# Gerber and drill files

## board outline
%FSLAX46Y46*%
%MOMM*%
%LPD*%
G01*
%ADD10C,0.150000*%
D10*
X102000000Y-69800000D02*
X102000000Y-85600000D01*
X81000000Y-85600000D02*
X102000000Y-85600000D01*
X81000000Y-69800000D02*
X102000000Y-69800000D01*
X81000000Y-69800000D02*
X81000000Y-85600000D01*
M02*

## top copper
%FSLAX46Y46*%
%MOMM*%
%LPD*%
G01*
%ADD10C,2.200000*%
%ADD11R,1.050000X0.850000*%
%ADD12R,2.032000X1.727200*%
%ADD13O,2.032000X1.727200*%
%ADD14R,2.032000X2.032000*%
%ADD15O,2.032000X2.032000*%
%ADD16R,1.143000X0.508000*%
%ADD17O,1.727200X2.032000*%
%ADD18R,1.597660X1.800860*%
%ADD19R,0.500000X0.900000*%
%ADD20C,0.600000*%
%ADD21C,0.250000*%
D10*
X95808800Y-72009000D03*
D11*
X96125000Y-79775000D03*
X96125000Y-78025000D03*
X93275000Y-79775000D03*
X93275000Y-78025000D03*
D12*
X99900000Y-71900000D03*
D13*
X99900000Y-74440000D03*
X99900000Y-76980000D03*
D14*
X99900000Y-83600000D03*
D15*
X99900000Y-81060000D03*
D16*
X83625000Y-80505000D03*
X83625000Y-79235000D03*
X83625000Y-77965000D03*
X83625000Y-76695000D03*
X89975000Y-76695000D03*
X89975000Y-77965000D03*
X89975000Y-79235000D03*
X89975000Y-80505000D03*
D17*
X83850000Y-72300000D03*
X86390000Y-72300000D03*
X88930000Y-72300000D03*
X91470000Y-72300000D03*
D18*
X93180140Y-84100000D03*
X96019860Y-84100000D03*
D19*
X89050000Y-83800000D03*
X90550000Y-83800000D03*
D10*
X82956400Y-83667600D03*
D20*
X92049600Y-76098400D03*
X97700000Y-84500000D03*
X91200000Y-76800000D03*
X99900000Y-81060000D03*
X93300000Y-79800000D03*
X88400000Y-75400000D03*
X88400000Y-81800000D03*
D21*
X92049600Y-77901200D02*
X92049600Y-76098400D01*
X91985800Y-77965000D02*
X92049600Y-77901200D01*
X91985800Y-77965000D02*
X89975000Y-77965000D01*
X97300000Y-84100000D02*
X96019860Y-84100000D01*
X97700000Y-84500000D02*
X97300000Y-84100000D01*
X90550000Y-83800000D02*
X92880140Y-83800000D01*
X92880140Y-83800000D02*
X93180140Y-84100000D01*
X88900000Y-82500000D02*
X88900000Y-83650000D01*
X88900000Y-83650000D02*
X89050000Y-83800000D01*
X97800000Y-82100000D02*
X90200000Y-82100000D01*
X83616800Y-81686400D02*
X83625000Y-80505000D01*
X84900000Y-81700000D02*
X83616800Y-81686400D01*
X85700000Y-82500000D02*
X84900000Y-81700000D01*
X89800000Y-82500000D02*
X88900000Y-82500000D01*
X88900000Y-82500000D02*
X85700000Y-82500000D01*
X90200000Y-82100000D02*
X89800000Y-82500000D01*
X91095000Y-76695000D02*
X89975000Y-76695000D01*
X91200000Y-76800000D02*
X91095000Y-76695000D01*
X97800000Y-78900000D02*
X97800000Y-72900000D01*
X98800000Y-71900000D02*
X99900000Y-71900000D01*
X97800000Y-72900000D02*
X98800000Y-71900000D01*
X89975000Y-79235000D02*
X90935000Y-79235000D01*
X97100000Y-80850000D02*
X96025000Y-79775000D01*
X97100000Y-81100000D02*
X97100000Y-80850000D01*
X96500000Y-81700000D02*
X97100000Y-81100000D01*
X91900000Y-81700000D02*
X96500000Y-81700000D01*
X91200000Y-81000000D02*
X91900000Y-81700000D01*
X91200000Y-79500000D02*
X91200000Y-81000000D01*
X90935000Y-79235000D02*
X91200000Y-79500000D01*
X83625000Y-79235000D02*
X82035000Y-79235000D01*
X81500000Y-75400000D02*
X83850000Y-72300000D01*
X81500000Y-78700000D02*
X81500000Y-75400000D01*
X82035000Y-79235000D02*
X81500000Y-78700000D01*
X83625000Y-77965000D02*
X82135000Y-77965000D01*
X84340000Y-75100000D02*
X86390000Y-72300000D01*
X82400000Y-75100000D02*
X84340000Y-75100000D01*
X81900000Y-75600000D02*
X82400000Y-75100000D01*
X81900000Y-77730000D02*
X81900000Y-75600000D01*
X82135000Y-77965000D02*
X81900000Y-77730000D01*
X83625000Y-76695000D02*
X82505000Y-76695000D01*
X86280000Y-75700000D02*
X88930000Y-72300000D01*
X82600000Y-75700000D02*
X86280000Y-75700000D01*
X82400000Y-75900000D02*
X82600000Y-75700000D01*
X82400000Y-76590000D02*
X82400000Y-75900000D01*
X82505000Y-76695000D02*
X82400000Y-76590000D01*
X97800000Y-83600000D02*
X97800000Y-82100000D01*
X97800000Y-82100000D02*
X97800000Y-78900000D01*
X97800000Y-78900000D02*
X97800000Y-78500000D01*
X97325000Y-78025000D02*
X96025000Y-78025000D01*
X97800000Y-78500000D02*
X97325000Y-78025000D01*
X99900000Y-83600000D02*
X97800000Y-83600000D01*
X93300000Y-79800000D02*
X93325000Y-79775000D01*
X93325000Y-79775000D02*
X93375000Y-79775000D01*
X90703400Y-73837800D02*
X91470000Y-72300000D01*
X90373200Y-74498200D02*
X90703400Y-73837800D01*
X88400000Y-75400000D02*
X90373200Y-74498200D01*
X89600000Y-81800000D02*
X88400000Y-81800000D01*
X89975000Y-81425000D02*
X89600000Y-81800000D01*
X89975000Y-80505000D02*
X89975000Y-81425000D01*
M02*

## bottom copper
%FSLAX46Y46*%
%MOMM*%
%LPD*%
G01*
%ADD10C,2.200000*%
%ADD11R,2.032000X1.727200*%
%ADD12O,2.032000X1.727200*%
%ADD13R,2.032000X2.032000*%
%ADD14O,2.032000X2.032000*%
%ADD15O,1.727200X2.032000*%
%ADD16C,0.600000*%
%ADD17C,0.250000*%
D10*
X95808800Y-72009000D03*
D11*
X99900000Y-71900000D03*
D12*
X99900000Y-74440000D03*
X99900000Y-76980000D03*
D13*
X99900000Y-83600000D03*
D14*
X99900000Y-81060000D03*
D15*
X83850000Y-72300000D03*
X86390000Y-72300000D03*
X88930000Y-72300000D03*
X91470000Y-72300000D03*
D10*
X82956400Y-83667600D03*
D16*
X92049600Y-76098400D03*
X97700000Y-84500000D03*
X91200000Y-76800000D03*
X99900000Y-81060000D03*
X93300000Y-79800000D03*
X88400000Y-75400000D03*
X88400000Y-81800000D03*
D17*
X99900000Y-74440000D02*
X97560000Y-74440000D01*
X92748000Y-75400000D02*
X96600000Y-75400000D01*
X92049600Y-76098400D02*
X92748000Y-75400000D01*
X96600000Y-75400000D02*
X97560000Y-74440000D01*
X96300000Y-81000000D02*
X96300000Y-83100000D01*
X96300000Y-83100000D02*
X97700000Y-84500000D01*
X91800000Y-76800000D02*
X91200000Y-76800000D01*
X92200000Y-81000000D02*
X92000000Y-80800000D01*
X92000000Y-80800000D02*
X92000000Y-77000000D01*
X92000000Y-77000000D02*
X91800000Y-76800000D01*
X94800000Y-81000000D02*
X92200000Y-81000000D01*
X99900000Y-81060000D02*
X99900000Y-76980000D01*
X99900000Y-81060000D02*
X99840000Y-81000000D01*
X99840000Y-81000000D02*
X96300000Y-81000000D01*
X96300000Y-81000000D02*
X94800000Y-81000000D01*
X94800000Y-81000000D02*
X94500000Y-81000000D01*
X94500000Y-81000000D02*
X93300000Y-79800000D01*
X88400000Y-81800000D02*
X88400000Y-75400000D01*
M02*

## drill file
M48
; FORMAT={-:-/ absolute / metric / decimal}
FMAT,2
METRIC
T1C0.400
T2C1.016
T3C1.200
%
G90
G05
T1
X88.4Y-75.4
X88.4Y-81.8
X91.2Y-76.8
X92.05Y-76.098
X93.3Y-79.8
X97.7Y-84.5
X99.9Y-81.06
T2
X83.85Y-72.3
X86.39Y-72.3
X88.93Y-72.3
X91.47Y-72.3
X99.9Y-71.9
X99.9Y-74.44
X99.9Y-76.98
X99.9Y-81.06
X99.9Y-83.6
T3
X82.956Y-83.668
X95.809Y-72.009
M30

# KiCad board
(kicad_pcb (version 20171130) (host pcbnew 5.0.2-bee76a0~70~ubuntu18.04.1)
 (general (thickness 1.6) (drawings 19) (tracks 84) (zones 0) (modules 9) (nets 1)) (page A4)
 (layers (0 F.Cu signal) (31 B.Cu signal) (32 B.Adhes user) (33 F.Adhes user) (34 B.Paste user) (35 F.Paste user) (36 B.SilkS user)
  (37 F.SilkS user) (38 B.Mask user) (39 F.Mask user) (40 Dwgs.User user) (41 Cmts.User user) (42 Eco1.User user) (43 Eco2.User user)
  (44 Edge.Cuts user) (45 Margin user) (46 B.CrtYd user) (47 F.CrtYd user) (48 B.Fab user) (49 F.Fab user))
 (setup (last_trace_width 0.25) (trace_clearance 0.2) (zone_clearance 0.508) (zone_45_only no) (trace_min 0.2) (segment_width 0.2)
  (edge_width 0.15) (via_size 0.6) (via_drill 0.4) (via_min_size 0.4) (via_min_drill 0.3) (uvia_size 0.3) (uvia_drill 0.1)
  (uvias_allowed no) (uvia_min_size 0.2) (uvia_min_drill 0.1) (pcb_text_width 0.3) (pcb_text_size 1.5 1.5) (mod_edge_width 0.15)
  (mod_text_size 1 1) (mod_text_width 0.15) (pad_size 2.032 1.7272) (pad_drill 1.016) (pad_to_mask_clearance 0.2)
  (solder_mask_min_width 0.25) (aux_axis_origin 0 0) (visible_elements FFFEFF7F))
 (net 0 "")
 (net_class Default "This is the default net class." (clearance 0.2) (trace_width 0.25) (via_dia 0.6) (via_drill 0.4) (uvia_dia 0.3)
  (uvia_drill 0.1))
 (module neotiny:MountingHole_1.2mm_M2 (layer F.Cu) (at 95.8088 72.009)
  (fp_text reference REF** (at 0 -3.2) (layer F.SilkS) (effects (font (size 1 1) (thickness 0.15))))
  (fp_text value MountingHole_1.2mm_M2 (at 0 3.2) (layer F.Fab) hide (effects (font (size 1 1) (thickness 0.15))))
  (pad "" np_thru_hole circle (at 0 0) (size 2.2 2.2) (drill 1.2) (layers *.Cu *.Mask)))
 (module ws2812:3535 (layer F.Cu) (at 94.7 78.9)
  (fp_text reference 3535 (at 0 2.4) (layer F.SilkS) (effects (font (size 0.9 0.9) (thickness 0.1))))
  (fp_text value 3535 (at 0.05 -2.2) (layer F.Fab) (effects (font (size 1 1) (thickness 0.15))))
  (pad IN smd rect (at 1.325 0.875) (size 1.05 0.85) (drill (offset 0.1 0)) (layers F.Cu F.Paste F.Mask))
  (pad VDD smd rect (at 1.325 -0.875) (size 1.05 0.85) (drill (offset 0.1 0)) (layers F.Cu F.Paste F.Mask))
  (pad GND smd rect (at -1.325 0.875) (size 1.05 0.85) (drill (offset -0.1 0)) (layers F.Cu F.Paste F.Mask))
  (pad OUT smd rect (at -1.325 -0.875) (size 1.05 0.85) (drill (offset -0.1 0)) (layers F.Cu F.Paste F.Mask)))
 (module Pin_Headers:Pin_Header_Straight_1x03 (layer F.Cu) (at 99.9 71.9)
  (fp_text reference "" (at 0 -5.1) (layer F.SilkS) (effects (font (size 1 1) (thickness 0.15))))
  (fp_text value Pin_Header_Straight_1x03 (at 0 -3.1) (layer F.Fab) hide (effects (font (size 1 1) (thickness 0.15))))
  (pad 1 thru_hole rect (at 0 0) (size 2.032 1.7272) (drill 1.016) (layers *.Cu *.Mask))
  (pad 2 thru_hole oval (at 0 2.54) (size 2.032 1.7272) (drill 1.016) (layers *.Cu *.Mask))
  (pad 3 thru_hole oval (at 0 5.08) (size 2.032 1.7272) (drill 1.016) (layers *.Cu *.Mask)))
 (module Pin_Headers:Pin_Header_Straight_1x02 (layer F.Cu) (at 99.9 83.6 180)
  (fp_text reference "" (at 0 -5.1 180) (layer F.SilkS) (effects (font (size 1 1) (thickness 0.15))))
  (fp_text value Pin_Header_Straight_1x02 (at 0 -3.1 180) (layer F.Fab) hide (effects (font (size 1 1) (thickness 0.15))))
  (pad 1 thru_hole rect (at 0 0 180) (size 2.032 2.032) (drill 1.016) (layers *.Cu *.Mask))
  (pad 2 thru_hole oval (at 0 2.54 180) (size 2.032 2.032) (drill 1.016) (layers *.Cu *.Mask)))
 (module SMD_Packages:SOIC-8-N (layer F.Cu) (at 86.8 78.6 90)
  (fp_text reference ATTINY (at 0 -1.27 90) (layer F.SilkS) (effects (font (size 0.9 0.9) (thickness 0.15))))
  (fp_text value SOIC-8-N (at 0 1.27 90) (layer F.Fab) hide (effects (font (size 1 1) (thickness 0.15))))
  (pad 8 smd rect (at -1.905 -3.175 90) (size 0.508 1.143) (layers F.Cu F.Paste F.Mask))
  (pad 7 smd rect (at -0.635 -3.175 90) (size 0.508 1.143) (layers F.Cu F.Paste F.Mask))
  (pad 6 smd rect (at 0.635 -3.175 90) (size 0.508 1.143) (layers F.Cu F.Paste F.Mask))
  (pad 5 smd rect (at 1.905 -3.175 90) (size 0.508 1.143) (layers F.Cu F.Paste F.Mask))
  (pad 4 smd rect (at 1.905 3.175 90) (size 0.508 1.143) (layers F.Cu F.Paste F.Mask))
  (pad 3 smd rect (at 0.635 3.175 90) (size 0.508 1.143) (layers F.Cu F.Paste F.Mask))
  (pad 2 smd rect (at -0.635 3.175 90) (size 0.508 1.143) (layers F.Cu F.Paste F.Mask))
  (pad 1 smd rect (at -1.905 3.175 90) (size 0.508 1.143) (layers F.Cu F.Paste F.Mask)))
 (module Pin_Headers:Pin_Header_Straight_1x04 (layer F.Cu) (at 83.85 72.3 90)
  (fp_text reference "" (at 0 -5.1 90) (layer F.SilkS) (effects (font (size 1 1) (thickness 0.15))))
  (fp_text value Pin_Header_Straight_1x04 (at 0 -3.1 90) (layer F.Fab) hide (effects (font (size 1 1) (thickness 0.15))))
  (pad 1 thru_hole oval (at 0 0 90) (size 2.032 1.7272) (drill 1.016) (layers *.Cu *.Mask))
  (pad 2 thru_hole oval (at 0 2.54 90) (size 2.032 1.7272) (drill 1.016) (layers *.Cu *.Mask))
  (pad 3 thru_hole oval (at 0 5.08 90) (size 2.032 1.7272) (drill 1.016) (layers *.Cu *.Mask))
  (pad 4 thru_hole oval (at 0 7.62 90) (size 2.032 1.7272) (drill 1.016) (layers *.Cu *.Mask)))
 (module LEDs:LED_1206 (layer F.Cu) (at 94.6 84.1 180)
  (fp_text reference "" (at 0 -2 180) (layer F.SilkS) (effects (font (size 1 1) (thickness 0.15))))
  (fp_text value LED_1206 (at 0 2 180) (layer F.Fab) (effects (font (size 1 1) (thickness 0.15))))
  (pad 2 smd rect (at 1.41986 0) (size 1.59766 1.80086) (layers F.Cu F.Paste F.Mask))
  (pad 1 smd rect (at -1.41986 0) (size 1.59766 1.80086) (layers F.Cu F.Paste F.Mask)))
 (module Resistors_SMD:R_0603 (layer F.Cu) (at 89.8 83.8)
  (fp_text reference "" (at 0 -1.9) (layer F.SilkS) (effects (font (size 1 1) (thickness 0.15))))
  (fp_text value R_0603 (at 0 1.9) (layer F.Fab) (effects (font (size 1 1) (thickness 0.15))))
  (pad 1 smd rect (at -0.75 0) (size 0.5 0.9) (layers F.Cu F.Paste F.Mask))
  (pad 2 smd rect (at 0.75 0) (size 0.5 0.9) (layers F.Cu F.Paste F.Mask)))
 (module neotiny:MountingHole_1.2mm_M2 (layer F.Cu) (at 82.9564 83.6676)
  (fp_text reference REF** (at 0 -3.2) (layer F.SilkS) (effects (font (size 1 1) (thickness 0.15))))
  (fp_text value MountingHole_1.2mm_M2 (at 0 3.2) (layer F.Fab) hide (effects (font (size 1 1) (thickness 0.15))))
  (pad "" np_thru_hole circle (at 0 0) (size 2.2 2.2) (drill 1.2) (layers *.Cu *.Mask)))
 (gr_line (start 102 69.8) (end 102 85.6) (angle 90) (layer Edge.Cuts) (width 0.15))
 (gr_line (start 81 85.6) (end 102 85.6) (angle 90) (layer Edge.Cuts) (width 0.15))
 (gr_line (start 81 69.8) (end 102 69.8) (angle 90) (layer Edge.Cuts) (width 0.15))
 (gr_line (start 81 69.8) (end 81 85.6) (angle 90) (layer Edge.Cuts) (width 0.15))
 (segment (start 99.9 74.44) (end 97.56 74.44) (width 0.25) (layer B.Cu) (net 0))
 (segment (start 92.748 75.4) (end 96.6 75.4) (width 0.25) (layer B.Cu) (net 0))
 (segment (start 92.0496 76.0984) (end 92.748 75.4) (width 0.25) (layer B.Cu) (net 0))
 (via (at 92.0496 76.0984) (size 0.6) (drill 0.4) (layers F.Cu B.Cu) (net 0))
 (segment (start 92.0496 77.9012) (end 92.0496 76.0984) (width 0.25) (layer F.Cu) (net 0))
 (segment (start 91.9858 77.965) (end 92.0496 77.9012) (width 0.25) (layer F.Cu) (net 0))
 (segment (start 91.9858 77.965) (end 89.975 77.965) (width 0.25) (layer F.Cu) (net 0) (status 800000))
 (segment (start 96.6 75.4) (end 97.56 74.44) (width 0.25) (layer B.Cu) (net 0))
 (segment (start 96.3 81) (end 96.3 83.1) (width 0.25) (layer B.Cu) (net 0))
 (segment (start 97.3 84.1) (end 96.01986 84.1) (width 0.25) (layer F.Cu) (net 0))
 (segment (start 97.7 84.5) (end 97.3 84.1) (width 0.25) (layer F.Cu) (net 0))
 (via (at 97.7 84.5) (size 0.6) (drill 0.4) (layers F.Cu B.Cu) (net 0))
 (segment (start 96.3 83.1) (end 97.7 84.5) (width 0.25) (layer B.Cu) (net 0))
 (segment (start 90.55 83.8) (end 92.88014 83.8) (width 0.25) (layer F.Cu) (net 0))
 (segment (start 92.88014 83.8) (end 93.18014 84.1) (width 0.25) (layer F.Cu) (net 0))
 (segment (start 88.9 82.5) (end 88.9 83.65) (width 0.25) (layer F.Cu) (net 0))
 (segment (start 88.9 83.65) (end 89.05 83.8) (width 0.25) (layer F.Cu) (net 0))
 (segment (start 97.8 82.1) (end 90.2 82.1) (width 0.25) (layer F.Cu) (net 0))
 (segment (start 83.6168 81.6864) (end 83.625 80.505) (width 0.25) (layer F.Cu) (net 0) (status 800000))
 (segment (start 84.9 81.7) (end 83.6168 81.6864) (width 0.25) (layer F.Cu) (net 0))
 (segment (start 85.7 82.5) (end 84.9 81.7) (width 0.25) (layer F.Cu) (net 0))
 (segment (start 89.8 82.5) (end 88.9 82.5) (width 0.25) (layer F.Cu) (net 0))
 (segment (start 88.9 82.5) (end 85.7 82.5) (width 0.25) (layer F.Cu) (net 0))
 (segment (start 90.2 82.1) (end 89.8 82.5) (width 0.25) (layer F.Cu) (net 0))
 (segment (start 91.8 76.8) (end 91.2 76.8) (width 0.25) (layer B.Cu) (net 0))
 (segment (start 92.2 81) (end 92 80.8) (width 0.25) (layer B.Cu) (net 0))
 (segment (start 92 80.8) (end 92 77) (width 0.25) (layer B.Cu) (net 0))
 (segment (start 92 77) (end 91.8 76.8) (width 0.25) (layer B.Cu) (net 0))
 (segment (start 94.8 81) (end 92.2 81) (width 0.25) (layer B.Cu) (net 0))
 (segment (start 91.095 76.695) (end 89.975 76.695) (width 0.25) (layer F.Cu) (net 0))
 (segment (start 91.2 76.8) (end 91.095 76.695) (width 0.25) (layer F.Cu) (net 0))
 (via (at 91.2 76.8) (size 0.6) (drill 0.4) (layers F.Cu B.Cu) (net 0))
 (segment (start 97.8 78.9) (end 97.8 72.9) (width 0.25) (layer F.Cu) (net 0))
 (segment (start 98.8 71.9) (end 99.9 71.9) (width 0.25) (layer F.Cu) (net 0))
 (segment (start 97.8 72.9) (end 98.8 71.9) (width 0.25) (layer F.Cu) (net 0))
 (segment (start 99.9 81.06) (end 99.9 76.98) (width 0.25) (layer B.Cu) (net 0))
 (segment (start 89.975 79.235) (end 90.935 79.235) (width 0.25) (layer F.Cu) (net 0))
 (segment (start 97.1 80.85) (end 96.025 79.775) (width 0.25) (layer F.Cu) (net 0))
 (segment (start 97.1 81.1) (end 97.1 80.85) (width 0.25) (layer F.Cu) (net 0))
 (segment (start 96.5 81.7) (end 97.1 81.1) (width 0.25) (layer F.Cu) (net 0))
 (segment (start 91.9 81.7) (end 96.5 81.7) (width 0.25) (layer F.Cu) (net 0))
 (segment (start 91.2 81) (end 91.9 81.7) (width 0.25) (layer F.Cu) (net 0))
 (segment (start 91.2 79.5) (end 91.2 81) (width 0.25) (layer F.Cu) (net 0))
 (segment (start 90.935 79.235) (end 91.2 79.5) (width 0.25) (layer F.Cu) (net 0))
 (segment (start 83.625 79.235) (end 82.035 79.235) (width 0.25) (layer F.Cu) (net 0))
 (segment (start 81.5 75.4) (end 83.85 72.3) (width 0.25) (layer F.Cu) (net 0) (status 20))
 (segment (start 81.5 78.7) (end 81.5 75.4) (width 0.25) (layer F.Cu) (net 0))
 (segment (start 82.035 79.235) (end 81.5 78.7) (width 0.25) (layer F.Cu) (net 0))
 (segment (start 83.625 77.965) (end 82.135 77.965) (width 0.25) (layer F.Cu) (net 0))
 (segment (start 84.34 75.1) (end 86.39 72.3) (width 0.25) (layer F.Cu) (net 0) (status 20))
 (segment (start 82.4 75.1) (end 84.34 75.1) (width 0.25) (layer F.Cu) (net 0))
 (segment (start 81.9 75.6) (end 82.4 75.1) (width 0.25) (layer F.Cu) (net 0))
 (segment (start 81.9 77.73) (end 81.9 75.6) (width 0.25) (layer F.Cu) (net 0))
 (segment (start 82.135 77.965) (end 81.9 77.73) (width 0.25) (layer F.Cu) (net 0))
 (segment (start 83.625 76.695) (end 82.505 76.695) (width 0.25) (layer F.Cu) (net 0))
 (segment (start 86.28 75.7) (end 88.93 72.3) (width 0.25) (layer F.Cu) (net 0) (status 20))
 (segment (start 82.6 75.7) (end 86.28 75.7) (width 0.25) (layer F.Cu) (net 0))
 (segment (start 82.4 75.9) (end 82.6 75.7) (width 0.25) (layer F.Cu) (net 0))
 (segment (start 82.4 76.59) (end 82.4 75.9) (width 0.25) (layer F.Cu) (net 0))
 (segment (start 82.505 76.695) (end 82.4 76.59) (width 0.25) (layer F.Cu) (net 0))
 (segment (start 97.8 83.6) (end 97.8 82.1) (width 0.25) (layer F.Cu) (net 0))
 (segment (start 97.8 82.1) (end 97.8 78.9) (width 0.25) (layer F.Cu) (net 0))
 (segment (start 97.8 78.9) (end 97.8 78.5) (width 0.25) (layer F.Cu) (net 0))
 (segment (start 97.325 78.025) (end 96.025 78.025) (width 0.25) (layer F.Cu) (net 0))
 (segment (start 97.8 78.5) (end 97.325 78.025) (width 0.25) (layer F.Cu) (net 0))
 (segment (start 99.9 83.6) (end 97.8 83.6) (width 0.25) (layer F.Cu) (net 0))
 (via (at 99.9 81.06) (size 0.6) (drill 0.4) (layers F.Cu B.Cu) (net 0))
 (segment (start 99.9 81.06) (end 99.84 81) (width 0.25) (layer B.Cu) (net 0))
 (segment (start 99.84 81) (end 96.3 81) (width 0.25) (layer B.Cu) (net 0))
 (segment (start 96.3 81) (end 94.8 81) (width 0.25) (layer B.Cu) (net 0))
 (segment (start 94.8 81) (end 94.5 81) (width 0.25) (layer B.Cu) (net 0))
 (segment (start 93.3 79.8) (end 93.325 79.775) (width 0.25) (layer F.Cu) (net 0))
 (via (at 93.3 79.8) (size 0.6) (drill 0.4) (layers F.Cu B.Cu) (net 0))
 (segment (start 94.5 81) (end 93.3 79.8) (width 0.25) (layer B.Cu) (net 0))
 (segment (start 93.325 79.775) (end 93.375 79.775) (width 0.25) (layer F.Cu) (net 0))
 (segment (start 90.7034 73.8378) (end 91.47 72.3) (width 0.25) (layer F.Cu) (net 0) (status 800020))
 (segment (start 90.3732 74.4982) (end 90.7034 73.8378) (width 0.25) (layer F.Cu) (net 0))
 (segment (start 88.4 75.4) (end 90.3732 74.4982) (width 0.25) (layer F.Cu) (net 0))
 (via (at 88.4 75.4) (size 0.6) (drill 0.4) (layers F.Cu B.Cu) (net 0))
 (segment (start 88.4 81.8) (end 88.4 75.4) (width 0.25) (layer B.Cu) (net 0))
 (via (at 88.4 81.8) (size 0.6) (drill 0.4) (layers F.Cu B.Cu) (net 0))
 (segment (start 89.6 81.8) (end 88.4 81.8) (width 0.25) (layer F.Cu) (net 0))
 (segment (start 89.975 81.425) (end 89.6 81.8) (width 0.25) (layer F.Cu) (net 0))
 (segment (start 89.975 80.505) (end 89.975 81.425) (width 0.25) (layer F.Cu) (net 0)))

